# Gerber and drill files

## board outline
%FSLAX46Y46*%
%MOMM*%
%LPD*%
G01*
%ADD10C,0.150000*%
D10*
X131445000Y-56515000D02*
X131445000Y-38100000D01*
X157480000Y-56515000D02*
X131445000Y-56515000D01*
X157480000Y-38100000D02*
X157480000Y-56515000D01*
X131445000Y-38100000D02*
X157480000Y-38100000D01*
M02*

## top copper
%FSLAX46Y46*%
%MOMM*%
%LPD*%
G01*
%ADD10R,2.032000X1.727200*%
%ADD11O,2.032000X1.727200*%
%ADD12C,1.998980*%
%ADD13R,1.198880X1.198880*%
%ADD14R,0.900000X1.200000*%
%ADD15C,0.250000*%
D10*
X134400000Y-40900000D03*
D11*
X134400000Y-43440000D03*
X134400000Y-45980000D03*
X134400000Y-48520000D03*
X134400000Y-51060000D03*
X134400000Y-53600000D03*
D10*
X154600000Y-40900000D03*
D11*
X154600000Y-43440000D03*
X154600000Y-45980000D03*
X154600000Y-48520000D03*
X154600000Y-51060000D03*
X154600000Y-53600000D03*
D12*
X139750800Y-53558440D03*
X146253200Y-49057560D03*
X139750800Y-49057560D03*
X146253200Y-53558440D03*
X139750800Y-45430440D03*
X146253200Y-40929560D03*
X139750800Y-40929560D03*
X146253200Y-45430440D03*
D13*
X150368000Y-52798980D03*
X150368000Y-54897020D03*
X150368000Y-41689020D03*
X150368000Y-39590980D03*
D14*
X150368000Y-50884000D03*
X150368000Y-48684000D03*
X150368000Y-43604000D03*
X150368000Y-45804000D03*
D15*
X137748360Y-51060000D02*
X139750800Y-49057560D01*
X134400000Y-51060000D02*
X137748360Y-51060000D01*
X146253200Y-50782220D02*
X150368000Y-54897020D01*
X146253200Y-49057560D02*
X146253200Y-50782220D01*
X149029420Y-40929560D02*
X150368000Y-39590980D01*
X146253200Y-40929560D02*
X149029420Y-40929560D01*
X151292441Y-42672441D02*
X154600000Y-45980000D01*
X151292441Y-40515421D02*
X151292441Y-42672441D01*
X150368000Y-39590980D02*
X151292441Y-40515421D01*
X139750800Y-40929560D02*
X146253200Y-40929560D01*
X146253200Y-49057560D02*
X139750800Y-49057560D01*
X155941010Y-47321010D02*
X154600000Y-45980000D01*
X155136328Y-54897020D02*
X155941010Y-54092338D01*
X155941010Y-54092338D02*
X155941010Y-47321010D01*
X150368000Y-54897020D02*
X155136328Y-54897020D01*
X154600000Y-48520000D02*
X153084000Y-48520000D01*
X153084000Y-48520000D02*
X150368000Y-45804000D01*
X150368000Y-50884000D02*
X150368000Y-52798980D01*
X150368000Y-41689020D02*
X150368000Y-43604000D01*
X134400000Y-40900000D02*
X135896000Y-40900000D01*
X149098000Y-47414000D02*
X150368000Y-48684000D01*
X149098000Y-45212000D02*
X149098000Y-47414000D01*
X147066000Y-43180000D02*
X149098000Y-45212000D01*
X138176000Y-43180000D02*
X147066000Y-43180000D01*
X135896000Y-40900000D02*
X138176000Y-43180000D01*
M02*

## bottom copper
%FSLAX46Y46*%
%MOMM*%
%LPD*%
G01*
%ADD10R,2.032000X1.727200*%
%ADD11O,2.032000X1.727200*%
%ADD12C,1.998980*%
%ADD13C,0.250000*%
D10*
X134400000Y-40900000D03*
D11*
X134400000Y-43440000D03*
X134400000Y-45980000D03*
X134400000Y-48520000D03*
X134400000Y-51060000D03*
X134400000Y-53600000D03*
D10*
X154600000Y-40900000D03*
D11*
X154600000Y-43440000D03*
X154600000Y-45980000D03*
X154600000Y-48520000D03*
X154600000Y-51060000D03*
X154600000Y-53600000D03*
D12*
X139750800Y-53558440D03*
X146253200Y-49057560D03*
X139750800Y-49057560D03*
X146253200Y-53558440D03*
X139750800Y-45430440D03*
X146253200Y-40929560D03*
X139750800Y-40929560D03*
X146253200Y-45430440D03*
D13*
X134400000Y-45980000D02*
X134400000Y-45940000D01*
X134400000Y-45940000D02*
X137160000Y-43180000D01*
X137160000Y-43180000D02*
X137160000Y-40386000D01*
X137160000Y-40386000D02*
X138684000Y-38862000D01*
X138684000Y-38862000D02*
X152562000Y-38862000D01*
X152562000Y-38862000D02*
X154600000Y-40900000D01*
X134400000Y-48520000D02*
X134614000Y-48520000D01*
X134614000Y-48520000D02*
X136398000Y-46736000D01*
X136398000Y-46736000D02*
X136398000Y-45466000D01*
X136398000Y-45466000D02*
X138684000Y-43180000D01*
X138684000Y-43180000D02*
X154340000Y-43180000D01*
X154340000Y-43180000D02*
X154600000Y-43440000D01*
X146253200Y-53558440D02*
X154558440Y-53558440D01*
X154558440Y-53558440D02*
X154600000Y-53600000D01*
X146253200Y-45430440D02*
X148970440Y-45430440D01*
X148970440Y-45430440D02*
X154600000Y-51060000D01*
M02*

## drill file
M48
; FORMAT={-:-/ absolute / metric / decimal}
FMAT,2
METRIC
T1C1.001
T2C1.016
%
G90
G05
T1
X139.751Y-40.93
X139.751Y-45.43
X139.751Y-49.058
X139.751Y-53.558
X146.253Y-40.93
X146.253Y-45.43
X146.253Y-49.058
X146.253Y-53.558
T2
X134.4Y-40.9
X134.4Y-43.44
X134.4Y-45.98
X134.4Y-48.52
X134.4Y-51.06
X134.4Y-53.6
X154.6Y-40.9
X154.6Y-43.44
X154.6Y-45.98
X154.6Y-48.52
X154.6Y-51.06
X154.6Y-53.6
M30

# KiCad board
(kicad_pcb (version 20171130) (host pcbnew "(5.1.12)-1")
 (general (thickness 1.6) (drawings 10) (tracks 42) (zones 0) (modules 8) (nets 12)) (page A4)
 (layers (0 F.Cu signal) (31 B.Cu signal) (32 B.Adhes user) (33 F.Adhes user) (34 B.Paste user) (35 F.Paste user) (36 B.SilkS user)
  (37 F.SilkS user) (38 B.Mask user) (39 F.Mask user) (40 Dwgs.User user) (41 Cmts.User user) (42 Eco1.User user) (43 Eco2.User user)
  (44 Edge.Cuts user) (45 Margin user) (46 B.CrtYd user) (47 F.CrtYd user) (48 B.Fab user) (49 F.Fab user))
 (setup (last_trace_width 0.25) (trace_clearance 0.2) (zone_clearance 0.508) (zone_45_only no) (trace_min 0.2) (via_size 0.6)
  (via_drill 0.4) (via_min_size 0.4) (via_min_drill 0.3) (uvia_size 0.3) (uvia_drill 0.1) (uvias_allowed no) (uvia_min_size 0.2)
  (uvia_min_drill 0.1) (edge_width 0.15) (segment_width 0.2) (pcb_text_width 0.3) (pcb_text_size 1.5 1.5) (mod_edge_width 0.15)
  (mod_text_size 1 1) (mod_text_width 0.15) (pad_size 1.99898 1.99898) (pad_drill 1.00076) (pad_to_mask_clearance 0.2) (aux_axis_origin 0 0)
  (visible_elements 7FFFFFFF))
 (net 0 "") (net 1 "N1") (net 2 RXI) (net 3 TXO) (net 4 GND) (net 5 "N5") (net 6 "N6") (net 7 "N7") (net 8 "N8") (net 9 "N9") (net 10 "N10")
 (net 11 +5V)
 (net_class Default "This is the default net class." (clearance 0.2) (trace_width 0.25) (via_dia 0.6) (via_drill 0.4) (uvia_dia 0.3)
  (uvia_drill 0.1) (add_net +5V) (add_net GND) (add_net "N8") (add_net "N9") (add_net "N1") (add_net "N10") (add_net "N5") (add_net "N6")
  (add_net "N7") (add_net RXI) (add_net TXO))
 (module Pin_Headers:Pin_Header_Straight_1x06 (layer F.Cu) (at 134.4 40.9)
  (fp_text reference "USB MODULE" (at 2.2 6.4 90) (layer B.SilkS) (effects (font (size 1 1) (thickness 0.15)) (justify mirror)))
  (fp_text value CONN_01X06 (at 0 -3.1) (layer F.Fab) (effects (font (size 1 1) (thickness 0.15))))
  (pad 1 thru_hole rect (at 0 0) (size 2.032 1.7272) (drill 1.016) (layers *.Cu *.Mask F.SilkS) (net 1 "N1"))
  (pad 2 thru_hole oval (at 0 2.54) (size 2.032 1.7272) (drill 1.016) (layers *.Cu *.Mask F.SilkS))
  (pad 3 thru_hole oval (at 0 5.08) (size 2.032 1.7272) (drill 1.016) (layers *.Cu *.Mask F.SilkS) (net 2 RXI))
  (pad 4 thru_hole oval (at 0 7.62) (size 2.032 1.7272) (drill 1.016) (layers *.Cu *.Mask F.SilkS) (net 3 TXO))
  (pad 5 thru_hole oval (at 0 10.16) (size 2.032 1.7272) (drill 1.016) (layers *.Cu *.Mask F.SilkS) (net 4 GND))
  (pad 6 thru_hole oval (at 0 12.7) (size 2.032 1.7272) (drill 1.016) (layers *.Cu *.Mask F.SilkS)))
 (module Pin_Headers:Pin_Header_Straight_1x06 (layer F.Cu) (at 154.6 40.9)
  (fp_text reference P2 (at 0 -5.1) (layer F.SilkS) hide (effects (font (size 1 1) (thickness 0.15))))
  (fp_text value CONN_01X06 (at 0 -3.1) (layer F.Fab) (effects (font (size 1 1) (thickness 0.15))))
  (pad 1 thru_hole rect (at 0 0) (size 2.032 1.7272) (drill 1.016) (layers *.Cu *.Mask F.SilkS) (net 2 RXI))
  (pad 2 thru_hole oval (at 0 2.54) (size 2.032 1.7272) (drill 1.016) (layers *.Cu *.Mask F.SilkS) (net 3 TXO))
  (pad 3 thru_hole oval (at 0 5.08) (size 2.032 1.7272) (drill 1.016) (layers *.Cu *.Mask F.SilkS) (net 4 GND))
  (pad 4 thru_hole oval (at 0 7.62) (size 2.032 1.7272) (drill 1.016) (layers *.Cu *.Mask F.SilkS) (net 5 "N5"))
  (pad 5 thru_hole oval (at 0 10.16) (size 2.032 1.7272) (drill 1.016) (layers *.Cu *.Mask F.SilkS) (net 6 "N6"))
  (pad 6 thru_hole oval (at 0 12.7) (size 2.032 1.7272) (drill 1.016) (layers *.Cu *.Mask F.SilkS) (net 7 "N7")))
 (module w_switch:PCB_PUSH (layer F.Cu) (at 143.002 51.308 90)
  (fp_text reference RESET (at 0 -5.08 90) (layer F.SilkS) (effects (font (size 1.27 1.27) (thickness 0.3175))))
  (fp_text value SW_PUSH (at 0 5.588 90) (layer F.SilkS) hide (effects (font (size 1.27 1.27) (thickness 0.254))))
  (pad 1 thru_hole circle (at -2.25044 -3.2512 90) (size 1.99898 1.99898) (drill 1.00076) (layers *.Cu *.Mask F.SilkS))
  (pad 2 thru_hole circle (at 2.25044 3.2512 90) (size 1.99898 1.99898) (drill 1.00076) (layers *.Cu *.Mask F.SilkS) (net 4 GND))
  (pad 4 thru_hole circle (at 2.25044 -3.2512 90) (size 1.99898 1.99898) (drill 1.00076) (layers *.Cu *.Mask F.SilkS) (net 4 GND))
  (pad 3 thru_hole circle (at -2.25044 3.2512 90) (size 1.99898 1.99898) (drill 1.00076) (layers *.Cu *.Mask F.SilkS) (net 7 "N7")))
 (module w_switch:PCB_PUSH (layer F.Cu) (at 143.002 43.18 90)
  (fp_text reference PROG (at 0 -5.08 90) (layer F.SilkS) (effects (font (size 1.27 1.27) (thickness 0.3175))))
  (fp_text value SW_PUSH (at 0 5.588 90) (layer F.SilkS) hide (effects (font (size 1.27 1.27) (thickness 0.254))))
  (pad 1 thru_hole circle (at -2.25044 -3.2512 90) (size 1.99898 1.99898) (drill 1.00076) (layers *.Cu *.Mask F.SilkS))
  (pad 2 thru_hole circle (at 2.25044 3.2512 90) (size 1.99898 1.99898) (drill 1.00076) (layers *.Cu *.Mask F.SilkS) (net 4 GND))
  (pad 4 thru_hole circle (at 2.25044 -3.2512 90) (size 1.99898 1.99898) (drill 1.00076) (layers *.Cu *.Mask F.SilkS) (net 4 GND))
  (pad 3 thru_hole circle (at -2.25044 3.2512 90) (size 1.99898 1.99898) (drill 1.00076) (layers *.Cu *.Mask F.SilkS) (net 6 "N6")))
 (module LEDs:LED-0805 (layer F.Cu) (at 150.368 53.848 90)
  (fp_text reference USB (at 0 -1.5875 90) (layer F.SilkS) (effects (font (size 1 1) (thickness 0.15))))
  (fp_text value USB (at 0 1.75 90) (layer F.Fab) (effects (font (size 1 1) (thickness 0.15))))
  (pad 2 smd rect (at 1.04902 0 270) (size 1.19888 1.19888) (layers F.Cu F.Paste F.Mask) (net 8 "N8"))
  (pad 1 smd rect (at -1.04902 0 270) (size 1.19888 1.19888) (layers F.Cu F.Paste F.Mask) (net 4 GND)))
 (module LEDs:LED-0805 (layer F.Cu) (at 150.368 40.64 270)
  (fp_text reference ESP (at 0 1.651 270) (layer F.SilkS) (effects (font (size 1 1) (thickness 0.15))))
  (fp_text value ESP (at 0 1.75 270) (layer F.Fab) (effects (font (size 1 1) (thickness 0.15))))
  (pad 2 smd rect (at 1.04902 0 90) (size 1.19888 1.19888) (layers F.Cu F.Paste F.Mask) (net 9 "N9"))
  (pad 1 smd rect (at -1.04902 0 90) (size 1.19888 1.19888) (layers F.Cu F.Paste F.Mask) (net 4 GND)))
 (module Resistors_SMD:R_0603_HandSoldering (layer F.Cu) (at 150.368 49.784 90)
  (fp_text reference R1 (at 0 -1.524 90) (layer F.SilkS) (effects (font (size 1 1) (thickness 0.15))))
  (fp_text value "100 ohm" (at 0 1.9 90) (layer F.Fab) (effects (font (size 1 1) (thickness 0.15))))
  (pad 1 smd rect (at -1.1 0 90) (size 1.2 0.9) (layers F.Cu F.Paste F.Mask) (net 8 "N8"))
  (pad 2 smd rect (at 1.1 0 90) (size 1.2 0.9) (layers F.Cu F.Paste F.Mask) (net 1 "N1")))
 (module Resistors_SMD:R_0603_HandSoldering (layer F.Cu) (at 150.368 44.704 270)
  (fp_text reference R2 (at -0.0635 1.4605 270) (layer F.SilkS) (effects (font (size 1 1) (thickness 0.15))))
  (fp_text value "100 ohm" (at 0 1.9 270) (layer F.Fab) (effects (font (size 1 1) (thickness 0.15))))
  (pad 1 smd rect (at -1.1 0 270) (size 1.2 0.9) (layers F.Cu F.Paste F.Mask) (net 9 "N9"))
  (pad 2 smd rect (at 1.1 0 270) (size 1.2 0.9) (layers F.Cu F.Paste F.Mask) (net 5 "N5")))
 (gr_line (start 131.445 56.515) (end 131.445 38.1) (angle 90) (layer Edge.Cuts) (width 0.15))
 (gr_line (start 157.48 56.515) (end 131.445 56.515) (angle 90) (layer Edge.Cuts) (width 0.15))
 (gr_line (start 157.48 38.1) (end 157.48 56.515) (angle 90) (layer Edge.Cuts) (width 0.15))
 (gr_line (start 131.445 38.1) (end 157.48 38.1) (angle 90) (layer Edge.Cuts) (width 0.15))
 (segment (start 134.4 45.98) (end 134.4 45.94) (width 0.25) (layer B.Cu) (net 2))
 (segment (start 134.4 45.94) (end 137.16 43.18) (width 0.25) (layer B.Cu) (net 2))
 (segment (start 137.16 43.18) (end 137.16 40.386) (width 0.25) (layer B.Cu) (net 2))
 (segment (start 137.16 40.386) (end 138.684 38.862) (width 0.25) (layer B.Cu) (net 2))
 (segment (start 138.684 38.862) (end 152.562 38.862) (width 0.25) (layer B.Cu) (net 2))
 (segment (start 152.562 38.862) (end 154.6 40.9) (width 0.25) (layer B.Cu) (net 2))
 (segment (start 134.4 48.52) (end 134.614 48.52) (width 0.25) (layer B.Cu) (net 3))
 (segment (start 134.614 48.52) (end 136.398 46.736) (width 0.25) (layer B.Cu) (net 3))
 (segment (start 136.398 46.736) (end 136.398 45.466) (width 0.25) (layer B.Cu) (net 3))
 (segment (start 136.398 45.466) (end 138.684 43.18) (width 0.25) (layer B.Cu) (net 3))
 (segment (start 138.684 43.18) (end 154.34 43.18) (width 0.25) (layer B.Cu) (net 3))
 (segment (start 154.34 43.18) (end 154.6 43.44) (width 0.25) (layer B.Cu) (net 3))
 (segment (start 137.74836 51.06) (end 139.7508 49.05756) (width 0.25) (layer F.Cu) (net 4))
 (segment (start 134.4 51.06) (end 137.74836 51.06) (width 0.25) (layer F.Cu) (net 4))
 (segment (start 146.2532 50.78222) (end 150.368 54.89702) (width 0.25) (layer F.Cu) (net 4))
 (segment (start 146.2532 49.05756) (end 146.2532 50.78222) (width 0.25) (layer F.Cu) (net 4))
 (segment (start 149.02942 40.92956) (end 150.368 39.59098) (width 0.25) (layer F.Cu) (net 4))
 (segment (start 146.2532 40.92956) (end 149.02942 40.92956) (width 0.25) (layer F.Cu) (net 4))
 (segment (start 151.292441 42.672441) (end 154.6 45.98) (width 0.25) (layer F.Cu) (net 4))
 (segment (start 151.292441 40.515421) (end 151.292441 42.672441) (width 0.25) (layer F.Cu) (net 4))
 (segment (start 150.368 39.59098) (end 151.292441 40.515421) (width 0.25) (layer F.Cu) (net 4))
 (segment (start 139.7508 40.92956) (end 146.2532 40.92956) (width 0.25) (layer F.Cu) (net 4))
 (segment (start 146.2532 49.05756) (end 139.7508 49.05756) (width 0.25) (layer F.Cu) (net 4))
 (segment (start 155.94101 47.32101) (end 154.6 45.98) (width 0.25) (layer F.Cu) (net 4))
 (segment (start 155.136328 54.89702) (end 155.94101 54.092338) (width 0.25) (layer F.Cu) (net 4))
 (segment (start 155.94101 54.092338) (end 155.94101 47.32101) (width 0.25) (layer F.Cu) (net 4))
 (segment (start 150.368 54.89702) (end 155.136328 54.89702) (width 0.25) (layer F.Cu) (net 4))
 (segment (start 154.6 48.52) (end 153.084 48.52) (width 0.25) (layer F.Cu) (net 5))
 (segment (start 153.084 48.52) (end 150.368 45.804) (width 0.25) (layer F.Cu) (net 5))
 (segment (start 146.2532 53.55844) (end 154.55844 53.55844) (width 0.25) (layer B.Cu) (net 7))
 (segment (start 154.55844 53.55844) (end 154.6 53.6) (width 0.25) (layer B.Cu) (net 7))
 (segment (start 146.2532 45.43044) (end 148.97044 45.43044) (width 0.25) (layer B.Cu) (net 6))
 (segment (start 148.97044 45.43044) (end 154.6 51.06) (width 0.25) (layer B.Cu) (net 6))
 (segment (start 150.368 50.884) (end 150.368 52.79898) (width 0.25) (layer F.Cu) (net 8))
 (segment (start 150.368 41.68902) (end 150.368 43.604) (width 0.25) (layer F.Cu) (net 9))
 (segment (start 134.4 40.9) (end 135.896 40.9) (width 0.25) (layer F.Cu) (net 1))
 (segment (start 149.098 47.414) (end 150.368 48.684) (width 0.25) (layer F.Cu) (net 1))
 (segment (start 149.098 45.212) (end 149.098 47.414) (width 0.25) (layer F.Cu) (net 1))
 (segment (start 147.066 43.18) (end 149.098 45.212) (width 0.25) (layer F.Cu) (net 1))
 (segment (start 138.176 43.18) (end 147.066 43.18) (width 0.25) (layer F.Cu) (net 1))
 (segment (start 135.896 40.9) (end 138.176 43.18) (width 0.25) (layer F.Cu) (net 1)))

